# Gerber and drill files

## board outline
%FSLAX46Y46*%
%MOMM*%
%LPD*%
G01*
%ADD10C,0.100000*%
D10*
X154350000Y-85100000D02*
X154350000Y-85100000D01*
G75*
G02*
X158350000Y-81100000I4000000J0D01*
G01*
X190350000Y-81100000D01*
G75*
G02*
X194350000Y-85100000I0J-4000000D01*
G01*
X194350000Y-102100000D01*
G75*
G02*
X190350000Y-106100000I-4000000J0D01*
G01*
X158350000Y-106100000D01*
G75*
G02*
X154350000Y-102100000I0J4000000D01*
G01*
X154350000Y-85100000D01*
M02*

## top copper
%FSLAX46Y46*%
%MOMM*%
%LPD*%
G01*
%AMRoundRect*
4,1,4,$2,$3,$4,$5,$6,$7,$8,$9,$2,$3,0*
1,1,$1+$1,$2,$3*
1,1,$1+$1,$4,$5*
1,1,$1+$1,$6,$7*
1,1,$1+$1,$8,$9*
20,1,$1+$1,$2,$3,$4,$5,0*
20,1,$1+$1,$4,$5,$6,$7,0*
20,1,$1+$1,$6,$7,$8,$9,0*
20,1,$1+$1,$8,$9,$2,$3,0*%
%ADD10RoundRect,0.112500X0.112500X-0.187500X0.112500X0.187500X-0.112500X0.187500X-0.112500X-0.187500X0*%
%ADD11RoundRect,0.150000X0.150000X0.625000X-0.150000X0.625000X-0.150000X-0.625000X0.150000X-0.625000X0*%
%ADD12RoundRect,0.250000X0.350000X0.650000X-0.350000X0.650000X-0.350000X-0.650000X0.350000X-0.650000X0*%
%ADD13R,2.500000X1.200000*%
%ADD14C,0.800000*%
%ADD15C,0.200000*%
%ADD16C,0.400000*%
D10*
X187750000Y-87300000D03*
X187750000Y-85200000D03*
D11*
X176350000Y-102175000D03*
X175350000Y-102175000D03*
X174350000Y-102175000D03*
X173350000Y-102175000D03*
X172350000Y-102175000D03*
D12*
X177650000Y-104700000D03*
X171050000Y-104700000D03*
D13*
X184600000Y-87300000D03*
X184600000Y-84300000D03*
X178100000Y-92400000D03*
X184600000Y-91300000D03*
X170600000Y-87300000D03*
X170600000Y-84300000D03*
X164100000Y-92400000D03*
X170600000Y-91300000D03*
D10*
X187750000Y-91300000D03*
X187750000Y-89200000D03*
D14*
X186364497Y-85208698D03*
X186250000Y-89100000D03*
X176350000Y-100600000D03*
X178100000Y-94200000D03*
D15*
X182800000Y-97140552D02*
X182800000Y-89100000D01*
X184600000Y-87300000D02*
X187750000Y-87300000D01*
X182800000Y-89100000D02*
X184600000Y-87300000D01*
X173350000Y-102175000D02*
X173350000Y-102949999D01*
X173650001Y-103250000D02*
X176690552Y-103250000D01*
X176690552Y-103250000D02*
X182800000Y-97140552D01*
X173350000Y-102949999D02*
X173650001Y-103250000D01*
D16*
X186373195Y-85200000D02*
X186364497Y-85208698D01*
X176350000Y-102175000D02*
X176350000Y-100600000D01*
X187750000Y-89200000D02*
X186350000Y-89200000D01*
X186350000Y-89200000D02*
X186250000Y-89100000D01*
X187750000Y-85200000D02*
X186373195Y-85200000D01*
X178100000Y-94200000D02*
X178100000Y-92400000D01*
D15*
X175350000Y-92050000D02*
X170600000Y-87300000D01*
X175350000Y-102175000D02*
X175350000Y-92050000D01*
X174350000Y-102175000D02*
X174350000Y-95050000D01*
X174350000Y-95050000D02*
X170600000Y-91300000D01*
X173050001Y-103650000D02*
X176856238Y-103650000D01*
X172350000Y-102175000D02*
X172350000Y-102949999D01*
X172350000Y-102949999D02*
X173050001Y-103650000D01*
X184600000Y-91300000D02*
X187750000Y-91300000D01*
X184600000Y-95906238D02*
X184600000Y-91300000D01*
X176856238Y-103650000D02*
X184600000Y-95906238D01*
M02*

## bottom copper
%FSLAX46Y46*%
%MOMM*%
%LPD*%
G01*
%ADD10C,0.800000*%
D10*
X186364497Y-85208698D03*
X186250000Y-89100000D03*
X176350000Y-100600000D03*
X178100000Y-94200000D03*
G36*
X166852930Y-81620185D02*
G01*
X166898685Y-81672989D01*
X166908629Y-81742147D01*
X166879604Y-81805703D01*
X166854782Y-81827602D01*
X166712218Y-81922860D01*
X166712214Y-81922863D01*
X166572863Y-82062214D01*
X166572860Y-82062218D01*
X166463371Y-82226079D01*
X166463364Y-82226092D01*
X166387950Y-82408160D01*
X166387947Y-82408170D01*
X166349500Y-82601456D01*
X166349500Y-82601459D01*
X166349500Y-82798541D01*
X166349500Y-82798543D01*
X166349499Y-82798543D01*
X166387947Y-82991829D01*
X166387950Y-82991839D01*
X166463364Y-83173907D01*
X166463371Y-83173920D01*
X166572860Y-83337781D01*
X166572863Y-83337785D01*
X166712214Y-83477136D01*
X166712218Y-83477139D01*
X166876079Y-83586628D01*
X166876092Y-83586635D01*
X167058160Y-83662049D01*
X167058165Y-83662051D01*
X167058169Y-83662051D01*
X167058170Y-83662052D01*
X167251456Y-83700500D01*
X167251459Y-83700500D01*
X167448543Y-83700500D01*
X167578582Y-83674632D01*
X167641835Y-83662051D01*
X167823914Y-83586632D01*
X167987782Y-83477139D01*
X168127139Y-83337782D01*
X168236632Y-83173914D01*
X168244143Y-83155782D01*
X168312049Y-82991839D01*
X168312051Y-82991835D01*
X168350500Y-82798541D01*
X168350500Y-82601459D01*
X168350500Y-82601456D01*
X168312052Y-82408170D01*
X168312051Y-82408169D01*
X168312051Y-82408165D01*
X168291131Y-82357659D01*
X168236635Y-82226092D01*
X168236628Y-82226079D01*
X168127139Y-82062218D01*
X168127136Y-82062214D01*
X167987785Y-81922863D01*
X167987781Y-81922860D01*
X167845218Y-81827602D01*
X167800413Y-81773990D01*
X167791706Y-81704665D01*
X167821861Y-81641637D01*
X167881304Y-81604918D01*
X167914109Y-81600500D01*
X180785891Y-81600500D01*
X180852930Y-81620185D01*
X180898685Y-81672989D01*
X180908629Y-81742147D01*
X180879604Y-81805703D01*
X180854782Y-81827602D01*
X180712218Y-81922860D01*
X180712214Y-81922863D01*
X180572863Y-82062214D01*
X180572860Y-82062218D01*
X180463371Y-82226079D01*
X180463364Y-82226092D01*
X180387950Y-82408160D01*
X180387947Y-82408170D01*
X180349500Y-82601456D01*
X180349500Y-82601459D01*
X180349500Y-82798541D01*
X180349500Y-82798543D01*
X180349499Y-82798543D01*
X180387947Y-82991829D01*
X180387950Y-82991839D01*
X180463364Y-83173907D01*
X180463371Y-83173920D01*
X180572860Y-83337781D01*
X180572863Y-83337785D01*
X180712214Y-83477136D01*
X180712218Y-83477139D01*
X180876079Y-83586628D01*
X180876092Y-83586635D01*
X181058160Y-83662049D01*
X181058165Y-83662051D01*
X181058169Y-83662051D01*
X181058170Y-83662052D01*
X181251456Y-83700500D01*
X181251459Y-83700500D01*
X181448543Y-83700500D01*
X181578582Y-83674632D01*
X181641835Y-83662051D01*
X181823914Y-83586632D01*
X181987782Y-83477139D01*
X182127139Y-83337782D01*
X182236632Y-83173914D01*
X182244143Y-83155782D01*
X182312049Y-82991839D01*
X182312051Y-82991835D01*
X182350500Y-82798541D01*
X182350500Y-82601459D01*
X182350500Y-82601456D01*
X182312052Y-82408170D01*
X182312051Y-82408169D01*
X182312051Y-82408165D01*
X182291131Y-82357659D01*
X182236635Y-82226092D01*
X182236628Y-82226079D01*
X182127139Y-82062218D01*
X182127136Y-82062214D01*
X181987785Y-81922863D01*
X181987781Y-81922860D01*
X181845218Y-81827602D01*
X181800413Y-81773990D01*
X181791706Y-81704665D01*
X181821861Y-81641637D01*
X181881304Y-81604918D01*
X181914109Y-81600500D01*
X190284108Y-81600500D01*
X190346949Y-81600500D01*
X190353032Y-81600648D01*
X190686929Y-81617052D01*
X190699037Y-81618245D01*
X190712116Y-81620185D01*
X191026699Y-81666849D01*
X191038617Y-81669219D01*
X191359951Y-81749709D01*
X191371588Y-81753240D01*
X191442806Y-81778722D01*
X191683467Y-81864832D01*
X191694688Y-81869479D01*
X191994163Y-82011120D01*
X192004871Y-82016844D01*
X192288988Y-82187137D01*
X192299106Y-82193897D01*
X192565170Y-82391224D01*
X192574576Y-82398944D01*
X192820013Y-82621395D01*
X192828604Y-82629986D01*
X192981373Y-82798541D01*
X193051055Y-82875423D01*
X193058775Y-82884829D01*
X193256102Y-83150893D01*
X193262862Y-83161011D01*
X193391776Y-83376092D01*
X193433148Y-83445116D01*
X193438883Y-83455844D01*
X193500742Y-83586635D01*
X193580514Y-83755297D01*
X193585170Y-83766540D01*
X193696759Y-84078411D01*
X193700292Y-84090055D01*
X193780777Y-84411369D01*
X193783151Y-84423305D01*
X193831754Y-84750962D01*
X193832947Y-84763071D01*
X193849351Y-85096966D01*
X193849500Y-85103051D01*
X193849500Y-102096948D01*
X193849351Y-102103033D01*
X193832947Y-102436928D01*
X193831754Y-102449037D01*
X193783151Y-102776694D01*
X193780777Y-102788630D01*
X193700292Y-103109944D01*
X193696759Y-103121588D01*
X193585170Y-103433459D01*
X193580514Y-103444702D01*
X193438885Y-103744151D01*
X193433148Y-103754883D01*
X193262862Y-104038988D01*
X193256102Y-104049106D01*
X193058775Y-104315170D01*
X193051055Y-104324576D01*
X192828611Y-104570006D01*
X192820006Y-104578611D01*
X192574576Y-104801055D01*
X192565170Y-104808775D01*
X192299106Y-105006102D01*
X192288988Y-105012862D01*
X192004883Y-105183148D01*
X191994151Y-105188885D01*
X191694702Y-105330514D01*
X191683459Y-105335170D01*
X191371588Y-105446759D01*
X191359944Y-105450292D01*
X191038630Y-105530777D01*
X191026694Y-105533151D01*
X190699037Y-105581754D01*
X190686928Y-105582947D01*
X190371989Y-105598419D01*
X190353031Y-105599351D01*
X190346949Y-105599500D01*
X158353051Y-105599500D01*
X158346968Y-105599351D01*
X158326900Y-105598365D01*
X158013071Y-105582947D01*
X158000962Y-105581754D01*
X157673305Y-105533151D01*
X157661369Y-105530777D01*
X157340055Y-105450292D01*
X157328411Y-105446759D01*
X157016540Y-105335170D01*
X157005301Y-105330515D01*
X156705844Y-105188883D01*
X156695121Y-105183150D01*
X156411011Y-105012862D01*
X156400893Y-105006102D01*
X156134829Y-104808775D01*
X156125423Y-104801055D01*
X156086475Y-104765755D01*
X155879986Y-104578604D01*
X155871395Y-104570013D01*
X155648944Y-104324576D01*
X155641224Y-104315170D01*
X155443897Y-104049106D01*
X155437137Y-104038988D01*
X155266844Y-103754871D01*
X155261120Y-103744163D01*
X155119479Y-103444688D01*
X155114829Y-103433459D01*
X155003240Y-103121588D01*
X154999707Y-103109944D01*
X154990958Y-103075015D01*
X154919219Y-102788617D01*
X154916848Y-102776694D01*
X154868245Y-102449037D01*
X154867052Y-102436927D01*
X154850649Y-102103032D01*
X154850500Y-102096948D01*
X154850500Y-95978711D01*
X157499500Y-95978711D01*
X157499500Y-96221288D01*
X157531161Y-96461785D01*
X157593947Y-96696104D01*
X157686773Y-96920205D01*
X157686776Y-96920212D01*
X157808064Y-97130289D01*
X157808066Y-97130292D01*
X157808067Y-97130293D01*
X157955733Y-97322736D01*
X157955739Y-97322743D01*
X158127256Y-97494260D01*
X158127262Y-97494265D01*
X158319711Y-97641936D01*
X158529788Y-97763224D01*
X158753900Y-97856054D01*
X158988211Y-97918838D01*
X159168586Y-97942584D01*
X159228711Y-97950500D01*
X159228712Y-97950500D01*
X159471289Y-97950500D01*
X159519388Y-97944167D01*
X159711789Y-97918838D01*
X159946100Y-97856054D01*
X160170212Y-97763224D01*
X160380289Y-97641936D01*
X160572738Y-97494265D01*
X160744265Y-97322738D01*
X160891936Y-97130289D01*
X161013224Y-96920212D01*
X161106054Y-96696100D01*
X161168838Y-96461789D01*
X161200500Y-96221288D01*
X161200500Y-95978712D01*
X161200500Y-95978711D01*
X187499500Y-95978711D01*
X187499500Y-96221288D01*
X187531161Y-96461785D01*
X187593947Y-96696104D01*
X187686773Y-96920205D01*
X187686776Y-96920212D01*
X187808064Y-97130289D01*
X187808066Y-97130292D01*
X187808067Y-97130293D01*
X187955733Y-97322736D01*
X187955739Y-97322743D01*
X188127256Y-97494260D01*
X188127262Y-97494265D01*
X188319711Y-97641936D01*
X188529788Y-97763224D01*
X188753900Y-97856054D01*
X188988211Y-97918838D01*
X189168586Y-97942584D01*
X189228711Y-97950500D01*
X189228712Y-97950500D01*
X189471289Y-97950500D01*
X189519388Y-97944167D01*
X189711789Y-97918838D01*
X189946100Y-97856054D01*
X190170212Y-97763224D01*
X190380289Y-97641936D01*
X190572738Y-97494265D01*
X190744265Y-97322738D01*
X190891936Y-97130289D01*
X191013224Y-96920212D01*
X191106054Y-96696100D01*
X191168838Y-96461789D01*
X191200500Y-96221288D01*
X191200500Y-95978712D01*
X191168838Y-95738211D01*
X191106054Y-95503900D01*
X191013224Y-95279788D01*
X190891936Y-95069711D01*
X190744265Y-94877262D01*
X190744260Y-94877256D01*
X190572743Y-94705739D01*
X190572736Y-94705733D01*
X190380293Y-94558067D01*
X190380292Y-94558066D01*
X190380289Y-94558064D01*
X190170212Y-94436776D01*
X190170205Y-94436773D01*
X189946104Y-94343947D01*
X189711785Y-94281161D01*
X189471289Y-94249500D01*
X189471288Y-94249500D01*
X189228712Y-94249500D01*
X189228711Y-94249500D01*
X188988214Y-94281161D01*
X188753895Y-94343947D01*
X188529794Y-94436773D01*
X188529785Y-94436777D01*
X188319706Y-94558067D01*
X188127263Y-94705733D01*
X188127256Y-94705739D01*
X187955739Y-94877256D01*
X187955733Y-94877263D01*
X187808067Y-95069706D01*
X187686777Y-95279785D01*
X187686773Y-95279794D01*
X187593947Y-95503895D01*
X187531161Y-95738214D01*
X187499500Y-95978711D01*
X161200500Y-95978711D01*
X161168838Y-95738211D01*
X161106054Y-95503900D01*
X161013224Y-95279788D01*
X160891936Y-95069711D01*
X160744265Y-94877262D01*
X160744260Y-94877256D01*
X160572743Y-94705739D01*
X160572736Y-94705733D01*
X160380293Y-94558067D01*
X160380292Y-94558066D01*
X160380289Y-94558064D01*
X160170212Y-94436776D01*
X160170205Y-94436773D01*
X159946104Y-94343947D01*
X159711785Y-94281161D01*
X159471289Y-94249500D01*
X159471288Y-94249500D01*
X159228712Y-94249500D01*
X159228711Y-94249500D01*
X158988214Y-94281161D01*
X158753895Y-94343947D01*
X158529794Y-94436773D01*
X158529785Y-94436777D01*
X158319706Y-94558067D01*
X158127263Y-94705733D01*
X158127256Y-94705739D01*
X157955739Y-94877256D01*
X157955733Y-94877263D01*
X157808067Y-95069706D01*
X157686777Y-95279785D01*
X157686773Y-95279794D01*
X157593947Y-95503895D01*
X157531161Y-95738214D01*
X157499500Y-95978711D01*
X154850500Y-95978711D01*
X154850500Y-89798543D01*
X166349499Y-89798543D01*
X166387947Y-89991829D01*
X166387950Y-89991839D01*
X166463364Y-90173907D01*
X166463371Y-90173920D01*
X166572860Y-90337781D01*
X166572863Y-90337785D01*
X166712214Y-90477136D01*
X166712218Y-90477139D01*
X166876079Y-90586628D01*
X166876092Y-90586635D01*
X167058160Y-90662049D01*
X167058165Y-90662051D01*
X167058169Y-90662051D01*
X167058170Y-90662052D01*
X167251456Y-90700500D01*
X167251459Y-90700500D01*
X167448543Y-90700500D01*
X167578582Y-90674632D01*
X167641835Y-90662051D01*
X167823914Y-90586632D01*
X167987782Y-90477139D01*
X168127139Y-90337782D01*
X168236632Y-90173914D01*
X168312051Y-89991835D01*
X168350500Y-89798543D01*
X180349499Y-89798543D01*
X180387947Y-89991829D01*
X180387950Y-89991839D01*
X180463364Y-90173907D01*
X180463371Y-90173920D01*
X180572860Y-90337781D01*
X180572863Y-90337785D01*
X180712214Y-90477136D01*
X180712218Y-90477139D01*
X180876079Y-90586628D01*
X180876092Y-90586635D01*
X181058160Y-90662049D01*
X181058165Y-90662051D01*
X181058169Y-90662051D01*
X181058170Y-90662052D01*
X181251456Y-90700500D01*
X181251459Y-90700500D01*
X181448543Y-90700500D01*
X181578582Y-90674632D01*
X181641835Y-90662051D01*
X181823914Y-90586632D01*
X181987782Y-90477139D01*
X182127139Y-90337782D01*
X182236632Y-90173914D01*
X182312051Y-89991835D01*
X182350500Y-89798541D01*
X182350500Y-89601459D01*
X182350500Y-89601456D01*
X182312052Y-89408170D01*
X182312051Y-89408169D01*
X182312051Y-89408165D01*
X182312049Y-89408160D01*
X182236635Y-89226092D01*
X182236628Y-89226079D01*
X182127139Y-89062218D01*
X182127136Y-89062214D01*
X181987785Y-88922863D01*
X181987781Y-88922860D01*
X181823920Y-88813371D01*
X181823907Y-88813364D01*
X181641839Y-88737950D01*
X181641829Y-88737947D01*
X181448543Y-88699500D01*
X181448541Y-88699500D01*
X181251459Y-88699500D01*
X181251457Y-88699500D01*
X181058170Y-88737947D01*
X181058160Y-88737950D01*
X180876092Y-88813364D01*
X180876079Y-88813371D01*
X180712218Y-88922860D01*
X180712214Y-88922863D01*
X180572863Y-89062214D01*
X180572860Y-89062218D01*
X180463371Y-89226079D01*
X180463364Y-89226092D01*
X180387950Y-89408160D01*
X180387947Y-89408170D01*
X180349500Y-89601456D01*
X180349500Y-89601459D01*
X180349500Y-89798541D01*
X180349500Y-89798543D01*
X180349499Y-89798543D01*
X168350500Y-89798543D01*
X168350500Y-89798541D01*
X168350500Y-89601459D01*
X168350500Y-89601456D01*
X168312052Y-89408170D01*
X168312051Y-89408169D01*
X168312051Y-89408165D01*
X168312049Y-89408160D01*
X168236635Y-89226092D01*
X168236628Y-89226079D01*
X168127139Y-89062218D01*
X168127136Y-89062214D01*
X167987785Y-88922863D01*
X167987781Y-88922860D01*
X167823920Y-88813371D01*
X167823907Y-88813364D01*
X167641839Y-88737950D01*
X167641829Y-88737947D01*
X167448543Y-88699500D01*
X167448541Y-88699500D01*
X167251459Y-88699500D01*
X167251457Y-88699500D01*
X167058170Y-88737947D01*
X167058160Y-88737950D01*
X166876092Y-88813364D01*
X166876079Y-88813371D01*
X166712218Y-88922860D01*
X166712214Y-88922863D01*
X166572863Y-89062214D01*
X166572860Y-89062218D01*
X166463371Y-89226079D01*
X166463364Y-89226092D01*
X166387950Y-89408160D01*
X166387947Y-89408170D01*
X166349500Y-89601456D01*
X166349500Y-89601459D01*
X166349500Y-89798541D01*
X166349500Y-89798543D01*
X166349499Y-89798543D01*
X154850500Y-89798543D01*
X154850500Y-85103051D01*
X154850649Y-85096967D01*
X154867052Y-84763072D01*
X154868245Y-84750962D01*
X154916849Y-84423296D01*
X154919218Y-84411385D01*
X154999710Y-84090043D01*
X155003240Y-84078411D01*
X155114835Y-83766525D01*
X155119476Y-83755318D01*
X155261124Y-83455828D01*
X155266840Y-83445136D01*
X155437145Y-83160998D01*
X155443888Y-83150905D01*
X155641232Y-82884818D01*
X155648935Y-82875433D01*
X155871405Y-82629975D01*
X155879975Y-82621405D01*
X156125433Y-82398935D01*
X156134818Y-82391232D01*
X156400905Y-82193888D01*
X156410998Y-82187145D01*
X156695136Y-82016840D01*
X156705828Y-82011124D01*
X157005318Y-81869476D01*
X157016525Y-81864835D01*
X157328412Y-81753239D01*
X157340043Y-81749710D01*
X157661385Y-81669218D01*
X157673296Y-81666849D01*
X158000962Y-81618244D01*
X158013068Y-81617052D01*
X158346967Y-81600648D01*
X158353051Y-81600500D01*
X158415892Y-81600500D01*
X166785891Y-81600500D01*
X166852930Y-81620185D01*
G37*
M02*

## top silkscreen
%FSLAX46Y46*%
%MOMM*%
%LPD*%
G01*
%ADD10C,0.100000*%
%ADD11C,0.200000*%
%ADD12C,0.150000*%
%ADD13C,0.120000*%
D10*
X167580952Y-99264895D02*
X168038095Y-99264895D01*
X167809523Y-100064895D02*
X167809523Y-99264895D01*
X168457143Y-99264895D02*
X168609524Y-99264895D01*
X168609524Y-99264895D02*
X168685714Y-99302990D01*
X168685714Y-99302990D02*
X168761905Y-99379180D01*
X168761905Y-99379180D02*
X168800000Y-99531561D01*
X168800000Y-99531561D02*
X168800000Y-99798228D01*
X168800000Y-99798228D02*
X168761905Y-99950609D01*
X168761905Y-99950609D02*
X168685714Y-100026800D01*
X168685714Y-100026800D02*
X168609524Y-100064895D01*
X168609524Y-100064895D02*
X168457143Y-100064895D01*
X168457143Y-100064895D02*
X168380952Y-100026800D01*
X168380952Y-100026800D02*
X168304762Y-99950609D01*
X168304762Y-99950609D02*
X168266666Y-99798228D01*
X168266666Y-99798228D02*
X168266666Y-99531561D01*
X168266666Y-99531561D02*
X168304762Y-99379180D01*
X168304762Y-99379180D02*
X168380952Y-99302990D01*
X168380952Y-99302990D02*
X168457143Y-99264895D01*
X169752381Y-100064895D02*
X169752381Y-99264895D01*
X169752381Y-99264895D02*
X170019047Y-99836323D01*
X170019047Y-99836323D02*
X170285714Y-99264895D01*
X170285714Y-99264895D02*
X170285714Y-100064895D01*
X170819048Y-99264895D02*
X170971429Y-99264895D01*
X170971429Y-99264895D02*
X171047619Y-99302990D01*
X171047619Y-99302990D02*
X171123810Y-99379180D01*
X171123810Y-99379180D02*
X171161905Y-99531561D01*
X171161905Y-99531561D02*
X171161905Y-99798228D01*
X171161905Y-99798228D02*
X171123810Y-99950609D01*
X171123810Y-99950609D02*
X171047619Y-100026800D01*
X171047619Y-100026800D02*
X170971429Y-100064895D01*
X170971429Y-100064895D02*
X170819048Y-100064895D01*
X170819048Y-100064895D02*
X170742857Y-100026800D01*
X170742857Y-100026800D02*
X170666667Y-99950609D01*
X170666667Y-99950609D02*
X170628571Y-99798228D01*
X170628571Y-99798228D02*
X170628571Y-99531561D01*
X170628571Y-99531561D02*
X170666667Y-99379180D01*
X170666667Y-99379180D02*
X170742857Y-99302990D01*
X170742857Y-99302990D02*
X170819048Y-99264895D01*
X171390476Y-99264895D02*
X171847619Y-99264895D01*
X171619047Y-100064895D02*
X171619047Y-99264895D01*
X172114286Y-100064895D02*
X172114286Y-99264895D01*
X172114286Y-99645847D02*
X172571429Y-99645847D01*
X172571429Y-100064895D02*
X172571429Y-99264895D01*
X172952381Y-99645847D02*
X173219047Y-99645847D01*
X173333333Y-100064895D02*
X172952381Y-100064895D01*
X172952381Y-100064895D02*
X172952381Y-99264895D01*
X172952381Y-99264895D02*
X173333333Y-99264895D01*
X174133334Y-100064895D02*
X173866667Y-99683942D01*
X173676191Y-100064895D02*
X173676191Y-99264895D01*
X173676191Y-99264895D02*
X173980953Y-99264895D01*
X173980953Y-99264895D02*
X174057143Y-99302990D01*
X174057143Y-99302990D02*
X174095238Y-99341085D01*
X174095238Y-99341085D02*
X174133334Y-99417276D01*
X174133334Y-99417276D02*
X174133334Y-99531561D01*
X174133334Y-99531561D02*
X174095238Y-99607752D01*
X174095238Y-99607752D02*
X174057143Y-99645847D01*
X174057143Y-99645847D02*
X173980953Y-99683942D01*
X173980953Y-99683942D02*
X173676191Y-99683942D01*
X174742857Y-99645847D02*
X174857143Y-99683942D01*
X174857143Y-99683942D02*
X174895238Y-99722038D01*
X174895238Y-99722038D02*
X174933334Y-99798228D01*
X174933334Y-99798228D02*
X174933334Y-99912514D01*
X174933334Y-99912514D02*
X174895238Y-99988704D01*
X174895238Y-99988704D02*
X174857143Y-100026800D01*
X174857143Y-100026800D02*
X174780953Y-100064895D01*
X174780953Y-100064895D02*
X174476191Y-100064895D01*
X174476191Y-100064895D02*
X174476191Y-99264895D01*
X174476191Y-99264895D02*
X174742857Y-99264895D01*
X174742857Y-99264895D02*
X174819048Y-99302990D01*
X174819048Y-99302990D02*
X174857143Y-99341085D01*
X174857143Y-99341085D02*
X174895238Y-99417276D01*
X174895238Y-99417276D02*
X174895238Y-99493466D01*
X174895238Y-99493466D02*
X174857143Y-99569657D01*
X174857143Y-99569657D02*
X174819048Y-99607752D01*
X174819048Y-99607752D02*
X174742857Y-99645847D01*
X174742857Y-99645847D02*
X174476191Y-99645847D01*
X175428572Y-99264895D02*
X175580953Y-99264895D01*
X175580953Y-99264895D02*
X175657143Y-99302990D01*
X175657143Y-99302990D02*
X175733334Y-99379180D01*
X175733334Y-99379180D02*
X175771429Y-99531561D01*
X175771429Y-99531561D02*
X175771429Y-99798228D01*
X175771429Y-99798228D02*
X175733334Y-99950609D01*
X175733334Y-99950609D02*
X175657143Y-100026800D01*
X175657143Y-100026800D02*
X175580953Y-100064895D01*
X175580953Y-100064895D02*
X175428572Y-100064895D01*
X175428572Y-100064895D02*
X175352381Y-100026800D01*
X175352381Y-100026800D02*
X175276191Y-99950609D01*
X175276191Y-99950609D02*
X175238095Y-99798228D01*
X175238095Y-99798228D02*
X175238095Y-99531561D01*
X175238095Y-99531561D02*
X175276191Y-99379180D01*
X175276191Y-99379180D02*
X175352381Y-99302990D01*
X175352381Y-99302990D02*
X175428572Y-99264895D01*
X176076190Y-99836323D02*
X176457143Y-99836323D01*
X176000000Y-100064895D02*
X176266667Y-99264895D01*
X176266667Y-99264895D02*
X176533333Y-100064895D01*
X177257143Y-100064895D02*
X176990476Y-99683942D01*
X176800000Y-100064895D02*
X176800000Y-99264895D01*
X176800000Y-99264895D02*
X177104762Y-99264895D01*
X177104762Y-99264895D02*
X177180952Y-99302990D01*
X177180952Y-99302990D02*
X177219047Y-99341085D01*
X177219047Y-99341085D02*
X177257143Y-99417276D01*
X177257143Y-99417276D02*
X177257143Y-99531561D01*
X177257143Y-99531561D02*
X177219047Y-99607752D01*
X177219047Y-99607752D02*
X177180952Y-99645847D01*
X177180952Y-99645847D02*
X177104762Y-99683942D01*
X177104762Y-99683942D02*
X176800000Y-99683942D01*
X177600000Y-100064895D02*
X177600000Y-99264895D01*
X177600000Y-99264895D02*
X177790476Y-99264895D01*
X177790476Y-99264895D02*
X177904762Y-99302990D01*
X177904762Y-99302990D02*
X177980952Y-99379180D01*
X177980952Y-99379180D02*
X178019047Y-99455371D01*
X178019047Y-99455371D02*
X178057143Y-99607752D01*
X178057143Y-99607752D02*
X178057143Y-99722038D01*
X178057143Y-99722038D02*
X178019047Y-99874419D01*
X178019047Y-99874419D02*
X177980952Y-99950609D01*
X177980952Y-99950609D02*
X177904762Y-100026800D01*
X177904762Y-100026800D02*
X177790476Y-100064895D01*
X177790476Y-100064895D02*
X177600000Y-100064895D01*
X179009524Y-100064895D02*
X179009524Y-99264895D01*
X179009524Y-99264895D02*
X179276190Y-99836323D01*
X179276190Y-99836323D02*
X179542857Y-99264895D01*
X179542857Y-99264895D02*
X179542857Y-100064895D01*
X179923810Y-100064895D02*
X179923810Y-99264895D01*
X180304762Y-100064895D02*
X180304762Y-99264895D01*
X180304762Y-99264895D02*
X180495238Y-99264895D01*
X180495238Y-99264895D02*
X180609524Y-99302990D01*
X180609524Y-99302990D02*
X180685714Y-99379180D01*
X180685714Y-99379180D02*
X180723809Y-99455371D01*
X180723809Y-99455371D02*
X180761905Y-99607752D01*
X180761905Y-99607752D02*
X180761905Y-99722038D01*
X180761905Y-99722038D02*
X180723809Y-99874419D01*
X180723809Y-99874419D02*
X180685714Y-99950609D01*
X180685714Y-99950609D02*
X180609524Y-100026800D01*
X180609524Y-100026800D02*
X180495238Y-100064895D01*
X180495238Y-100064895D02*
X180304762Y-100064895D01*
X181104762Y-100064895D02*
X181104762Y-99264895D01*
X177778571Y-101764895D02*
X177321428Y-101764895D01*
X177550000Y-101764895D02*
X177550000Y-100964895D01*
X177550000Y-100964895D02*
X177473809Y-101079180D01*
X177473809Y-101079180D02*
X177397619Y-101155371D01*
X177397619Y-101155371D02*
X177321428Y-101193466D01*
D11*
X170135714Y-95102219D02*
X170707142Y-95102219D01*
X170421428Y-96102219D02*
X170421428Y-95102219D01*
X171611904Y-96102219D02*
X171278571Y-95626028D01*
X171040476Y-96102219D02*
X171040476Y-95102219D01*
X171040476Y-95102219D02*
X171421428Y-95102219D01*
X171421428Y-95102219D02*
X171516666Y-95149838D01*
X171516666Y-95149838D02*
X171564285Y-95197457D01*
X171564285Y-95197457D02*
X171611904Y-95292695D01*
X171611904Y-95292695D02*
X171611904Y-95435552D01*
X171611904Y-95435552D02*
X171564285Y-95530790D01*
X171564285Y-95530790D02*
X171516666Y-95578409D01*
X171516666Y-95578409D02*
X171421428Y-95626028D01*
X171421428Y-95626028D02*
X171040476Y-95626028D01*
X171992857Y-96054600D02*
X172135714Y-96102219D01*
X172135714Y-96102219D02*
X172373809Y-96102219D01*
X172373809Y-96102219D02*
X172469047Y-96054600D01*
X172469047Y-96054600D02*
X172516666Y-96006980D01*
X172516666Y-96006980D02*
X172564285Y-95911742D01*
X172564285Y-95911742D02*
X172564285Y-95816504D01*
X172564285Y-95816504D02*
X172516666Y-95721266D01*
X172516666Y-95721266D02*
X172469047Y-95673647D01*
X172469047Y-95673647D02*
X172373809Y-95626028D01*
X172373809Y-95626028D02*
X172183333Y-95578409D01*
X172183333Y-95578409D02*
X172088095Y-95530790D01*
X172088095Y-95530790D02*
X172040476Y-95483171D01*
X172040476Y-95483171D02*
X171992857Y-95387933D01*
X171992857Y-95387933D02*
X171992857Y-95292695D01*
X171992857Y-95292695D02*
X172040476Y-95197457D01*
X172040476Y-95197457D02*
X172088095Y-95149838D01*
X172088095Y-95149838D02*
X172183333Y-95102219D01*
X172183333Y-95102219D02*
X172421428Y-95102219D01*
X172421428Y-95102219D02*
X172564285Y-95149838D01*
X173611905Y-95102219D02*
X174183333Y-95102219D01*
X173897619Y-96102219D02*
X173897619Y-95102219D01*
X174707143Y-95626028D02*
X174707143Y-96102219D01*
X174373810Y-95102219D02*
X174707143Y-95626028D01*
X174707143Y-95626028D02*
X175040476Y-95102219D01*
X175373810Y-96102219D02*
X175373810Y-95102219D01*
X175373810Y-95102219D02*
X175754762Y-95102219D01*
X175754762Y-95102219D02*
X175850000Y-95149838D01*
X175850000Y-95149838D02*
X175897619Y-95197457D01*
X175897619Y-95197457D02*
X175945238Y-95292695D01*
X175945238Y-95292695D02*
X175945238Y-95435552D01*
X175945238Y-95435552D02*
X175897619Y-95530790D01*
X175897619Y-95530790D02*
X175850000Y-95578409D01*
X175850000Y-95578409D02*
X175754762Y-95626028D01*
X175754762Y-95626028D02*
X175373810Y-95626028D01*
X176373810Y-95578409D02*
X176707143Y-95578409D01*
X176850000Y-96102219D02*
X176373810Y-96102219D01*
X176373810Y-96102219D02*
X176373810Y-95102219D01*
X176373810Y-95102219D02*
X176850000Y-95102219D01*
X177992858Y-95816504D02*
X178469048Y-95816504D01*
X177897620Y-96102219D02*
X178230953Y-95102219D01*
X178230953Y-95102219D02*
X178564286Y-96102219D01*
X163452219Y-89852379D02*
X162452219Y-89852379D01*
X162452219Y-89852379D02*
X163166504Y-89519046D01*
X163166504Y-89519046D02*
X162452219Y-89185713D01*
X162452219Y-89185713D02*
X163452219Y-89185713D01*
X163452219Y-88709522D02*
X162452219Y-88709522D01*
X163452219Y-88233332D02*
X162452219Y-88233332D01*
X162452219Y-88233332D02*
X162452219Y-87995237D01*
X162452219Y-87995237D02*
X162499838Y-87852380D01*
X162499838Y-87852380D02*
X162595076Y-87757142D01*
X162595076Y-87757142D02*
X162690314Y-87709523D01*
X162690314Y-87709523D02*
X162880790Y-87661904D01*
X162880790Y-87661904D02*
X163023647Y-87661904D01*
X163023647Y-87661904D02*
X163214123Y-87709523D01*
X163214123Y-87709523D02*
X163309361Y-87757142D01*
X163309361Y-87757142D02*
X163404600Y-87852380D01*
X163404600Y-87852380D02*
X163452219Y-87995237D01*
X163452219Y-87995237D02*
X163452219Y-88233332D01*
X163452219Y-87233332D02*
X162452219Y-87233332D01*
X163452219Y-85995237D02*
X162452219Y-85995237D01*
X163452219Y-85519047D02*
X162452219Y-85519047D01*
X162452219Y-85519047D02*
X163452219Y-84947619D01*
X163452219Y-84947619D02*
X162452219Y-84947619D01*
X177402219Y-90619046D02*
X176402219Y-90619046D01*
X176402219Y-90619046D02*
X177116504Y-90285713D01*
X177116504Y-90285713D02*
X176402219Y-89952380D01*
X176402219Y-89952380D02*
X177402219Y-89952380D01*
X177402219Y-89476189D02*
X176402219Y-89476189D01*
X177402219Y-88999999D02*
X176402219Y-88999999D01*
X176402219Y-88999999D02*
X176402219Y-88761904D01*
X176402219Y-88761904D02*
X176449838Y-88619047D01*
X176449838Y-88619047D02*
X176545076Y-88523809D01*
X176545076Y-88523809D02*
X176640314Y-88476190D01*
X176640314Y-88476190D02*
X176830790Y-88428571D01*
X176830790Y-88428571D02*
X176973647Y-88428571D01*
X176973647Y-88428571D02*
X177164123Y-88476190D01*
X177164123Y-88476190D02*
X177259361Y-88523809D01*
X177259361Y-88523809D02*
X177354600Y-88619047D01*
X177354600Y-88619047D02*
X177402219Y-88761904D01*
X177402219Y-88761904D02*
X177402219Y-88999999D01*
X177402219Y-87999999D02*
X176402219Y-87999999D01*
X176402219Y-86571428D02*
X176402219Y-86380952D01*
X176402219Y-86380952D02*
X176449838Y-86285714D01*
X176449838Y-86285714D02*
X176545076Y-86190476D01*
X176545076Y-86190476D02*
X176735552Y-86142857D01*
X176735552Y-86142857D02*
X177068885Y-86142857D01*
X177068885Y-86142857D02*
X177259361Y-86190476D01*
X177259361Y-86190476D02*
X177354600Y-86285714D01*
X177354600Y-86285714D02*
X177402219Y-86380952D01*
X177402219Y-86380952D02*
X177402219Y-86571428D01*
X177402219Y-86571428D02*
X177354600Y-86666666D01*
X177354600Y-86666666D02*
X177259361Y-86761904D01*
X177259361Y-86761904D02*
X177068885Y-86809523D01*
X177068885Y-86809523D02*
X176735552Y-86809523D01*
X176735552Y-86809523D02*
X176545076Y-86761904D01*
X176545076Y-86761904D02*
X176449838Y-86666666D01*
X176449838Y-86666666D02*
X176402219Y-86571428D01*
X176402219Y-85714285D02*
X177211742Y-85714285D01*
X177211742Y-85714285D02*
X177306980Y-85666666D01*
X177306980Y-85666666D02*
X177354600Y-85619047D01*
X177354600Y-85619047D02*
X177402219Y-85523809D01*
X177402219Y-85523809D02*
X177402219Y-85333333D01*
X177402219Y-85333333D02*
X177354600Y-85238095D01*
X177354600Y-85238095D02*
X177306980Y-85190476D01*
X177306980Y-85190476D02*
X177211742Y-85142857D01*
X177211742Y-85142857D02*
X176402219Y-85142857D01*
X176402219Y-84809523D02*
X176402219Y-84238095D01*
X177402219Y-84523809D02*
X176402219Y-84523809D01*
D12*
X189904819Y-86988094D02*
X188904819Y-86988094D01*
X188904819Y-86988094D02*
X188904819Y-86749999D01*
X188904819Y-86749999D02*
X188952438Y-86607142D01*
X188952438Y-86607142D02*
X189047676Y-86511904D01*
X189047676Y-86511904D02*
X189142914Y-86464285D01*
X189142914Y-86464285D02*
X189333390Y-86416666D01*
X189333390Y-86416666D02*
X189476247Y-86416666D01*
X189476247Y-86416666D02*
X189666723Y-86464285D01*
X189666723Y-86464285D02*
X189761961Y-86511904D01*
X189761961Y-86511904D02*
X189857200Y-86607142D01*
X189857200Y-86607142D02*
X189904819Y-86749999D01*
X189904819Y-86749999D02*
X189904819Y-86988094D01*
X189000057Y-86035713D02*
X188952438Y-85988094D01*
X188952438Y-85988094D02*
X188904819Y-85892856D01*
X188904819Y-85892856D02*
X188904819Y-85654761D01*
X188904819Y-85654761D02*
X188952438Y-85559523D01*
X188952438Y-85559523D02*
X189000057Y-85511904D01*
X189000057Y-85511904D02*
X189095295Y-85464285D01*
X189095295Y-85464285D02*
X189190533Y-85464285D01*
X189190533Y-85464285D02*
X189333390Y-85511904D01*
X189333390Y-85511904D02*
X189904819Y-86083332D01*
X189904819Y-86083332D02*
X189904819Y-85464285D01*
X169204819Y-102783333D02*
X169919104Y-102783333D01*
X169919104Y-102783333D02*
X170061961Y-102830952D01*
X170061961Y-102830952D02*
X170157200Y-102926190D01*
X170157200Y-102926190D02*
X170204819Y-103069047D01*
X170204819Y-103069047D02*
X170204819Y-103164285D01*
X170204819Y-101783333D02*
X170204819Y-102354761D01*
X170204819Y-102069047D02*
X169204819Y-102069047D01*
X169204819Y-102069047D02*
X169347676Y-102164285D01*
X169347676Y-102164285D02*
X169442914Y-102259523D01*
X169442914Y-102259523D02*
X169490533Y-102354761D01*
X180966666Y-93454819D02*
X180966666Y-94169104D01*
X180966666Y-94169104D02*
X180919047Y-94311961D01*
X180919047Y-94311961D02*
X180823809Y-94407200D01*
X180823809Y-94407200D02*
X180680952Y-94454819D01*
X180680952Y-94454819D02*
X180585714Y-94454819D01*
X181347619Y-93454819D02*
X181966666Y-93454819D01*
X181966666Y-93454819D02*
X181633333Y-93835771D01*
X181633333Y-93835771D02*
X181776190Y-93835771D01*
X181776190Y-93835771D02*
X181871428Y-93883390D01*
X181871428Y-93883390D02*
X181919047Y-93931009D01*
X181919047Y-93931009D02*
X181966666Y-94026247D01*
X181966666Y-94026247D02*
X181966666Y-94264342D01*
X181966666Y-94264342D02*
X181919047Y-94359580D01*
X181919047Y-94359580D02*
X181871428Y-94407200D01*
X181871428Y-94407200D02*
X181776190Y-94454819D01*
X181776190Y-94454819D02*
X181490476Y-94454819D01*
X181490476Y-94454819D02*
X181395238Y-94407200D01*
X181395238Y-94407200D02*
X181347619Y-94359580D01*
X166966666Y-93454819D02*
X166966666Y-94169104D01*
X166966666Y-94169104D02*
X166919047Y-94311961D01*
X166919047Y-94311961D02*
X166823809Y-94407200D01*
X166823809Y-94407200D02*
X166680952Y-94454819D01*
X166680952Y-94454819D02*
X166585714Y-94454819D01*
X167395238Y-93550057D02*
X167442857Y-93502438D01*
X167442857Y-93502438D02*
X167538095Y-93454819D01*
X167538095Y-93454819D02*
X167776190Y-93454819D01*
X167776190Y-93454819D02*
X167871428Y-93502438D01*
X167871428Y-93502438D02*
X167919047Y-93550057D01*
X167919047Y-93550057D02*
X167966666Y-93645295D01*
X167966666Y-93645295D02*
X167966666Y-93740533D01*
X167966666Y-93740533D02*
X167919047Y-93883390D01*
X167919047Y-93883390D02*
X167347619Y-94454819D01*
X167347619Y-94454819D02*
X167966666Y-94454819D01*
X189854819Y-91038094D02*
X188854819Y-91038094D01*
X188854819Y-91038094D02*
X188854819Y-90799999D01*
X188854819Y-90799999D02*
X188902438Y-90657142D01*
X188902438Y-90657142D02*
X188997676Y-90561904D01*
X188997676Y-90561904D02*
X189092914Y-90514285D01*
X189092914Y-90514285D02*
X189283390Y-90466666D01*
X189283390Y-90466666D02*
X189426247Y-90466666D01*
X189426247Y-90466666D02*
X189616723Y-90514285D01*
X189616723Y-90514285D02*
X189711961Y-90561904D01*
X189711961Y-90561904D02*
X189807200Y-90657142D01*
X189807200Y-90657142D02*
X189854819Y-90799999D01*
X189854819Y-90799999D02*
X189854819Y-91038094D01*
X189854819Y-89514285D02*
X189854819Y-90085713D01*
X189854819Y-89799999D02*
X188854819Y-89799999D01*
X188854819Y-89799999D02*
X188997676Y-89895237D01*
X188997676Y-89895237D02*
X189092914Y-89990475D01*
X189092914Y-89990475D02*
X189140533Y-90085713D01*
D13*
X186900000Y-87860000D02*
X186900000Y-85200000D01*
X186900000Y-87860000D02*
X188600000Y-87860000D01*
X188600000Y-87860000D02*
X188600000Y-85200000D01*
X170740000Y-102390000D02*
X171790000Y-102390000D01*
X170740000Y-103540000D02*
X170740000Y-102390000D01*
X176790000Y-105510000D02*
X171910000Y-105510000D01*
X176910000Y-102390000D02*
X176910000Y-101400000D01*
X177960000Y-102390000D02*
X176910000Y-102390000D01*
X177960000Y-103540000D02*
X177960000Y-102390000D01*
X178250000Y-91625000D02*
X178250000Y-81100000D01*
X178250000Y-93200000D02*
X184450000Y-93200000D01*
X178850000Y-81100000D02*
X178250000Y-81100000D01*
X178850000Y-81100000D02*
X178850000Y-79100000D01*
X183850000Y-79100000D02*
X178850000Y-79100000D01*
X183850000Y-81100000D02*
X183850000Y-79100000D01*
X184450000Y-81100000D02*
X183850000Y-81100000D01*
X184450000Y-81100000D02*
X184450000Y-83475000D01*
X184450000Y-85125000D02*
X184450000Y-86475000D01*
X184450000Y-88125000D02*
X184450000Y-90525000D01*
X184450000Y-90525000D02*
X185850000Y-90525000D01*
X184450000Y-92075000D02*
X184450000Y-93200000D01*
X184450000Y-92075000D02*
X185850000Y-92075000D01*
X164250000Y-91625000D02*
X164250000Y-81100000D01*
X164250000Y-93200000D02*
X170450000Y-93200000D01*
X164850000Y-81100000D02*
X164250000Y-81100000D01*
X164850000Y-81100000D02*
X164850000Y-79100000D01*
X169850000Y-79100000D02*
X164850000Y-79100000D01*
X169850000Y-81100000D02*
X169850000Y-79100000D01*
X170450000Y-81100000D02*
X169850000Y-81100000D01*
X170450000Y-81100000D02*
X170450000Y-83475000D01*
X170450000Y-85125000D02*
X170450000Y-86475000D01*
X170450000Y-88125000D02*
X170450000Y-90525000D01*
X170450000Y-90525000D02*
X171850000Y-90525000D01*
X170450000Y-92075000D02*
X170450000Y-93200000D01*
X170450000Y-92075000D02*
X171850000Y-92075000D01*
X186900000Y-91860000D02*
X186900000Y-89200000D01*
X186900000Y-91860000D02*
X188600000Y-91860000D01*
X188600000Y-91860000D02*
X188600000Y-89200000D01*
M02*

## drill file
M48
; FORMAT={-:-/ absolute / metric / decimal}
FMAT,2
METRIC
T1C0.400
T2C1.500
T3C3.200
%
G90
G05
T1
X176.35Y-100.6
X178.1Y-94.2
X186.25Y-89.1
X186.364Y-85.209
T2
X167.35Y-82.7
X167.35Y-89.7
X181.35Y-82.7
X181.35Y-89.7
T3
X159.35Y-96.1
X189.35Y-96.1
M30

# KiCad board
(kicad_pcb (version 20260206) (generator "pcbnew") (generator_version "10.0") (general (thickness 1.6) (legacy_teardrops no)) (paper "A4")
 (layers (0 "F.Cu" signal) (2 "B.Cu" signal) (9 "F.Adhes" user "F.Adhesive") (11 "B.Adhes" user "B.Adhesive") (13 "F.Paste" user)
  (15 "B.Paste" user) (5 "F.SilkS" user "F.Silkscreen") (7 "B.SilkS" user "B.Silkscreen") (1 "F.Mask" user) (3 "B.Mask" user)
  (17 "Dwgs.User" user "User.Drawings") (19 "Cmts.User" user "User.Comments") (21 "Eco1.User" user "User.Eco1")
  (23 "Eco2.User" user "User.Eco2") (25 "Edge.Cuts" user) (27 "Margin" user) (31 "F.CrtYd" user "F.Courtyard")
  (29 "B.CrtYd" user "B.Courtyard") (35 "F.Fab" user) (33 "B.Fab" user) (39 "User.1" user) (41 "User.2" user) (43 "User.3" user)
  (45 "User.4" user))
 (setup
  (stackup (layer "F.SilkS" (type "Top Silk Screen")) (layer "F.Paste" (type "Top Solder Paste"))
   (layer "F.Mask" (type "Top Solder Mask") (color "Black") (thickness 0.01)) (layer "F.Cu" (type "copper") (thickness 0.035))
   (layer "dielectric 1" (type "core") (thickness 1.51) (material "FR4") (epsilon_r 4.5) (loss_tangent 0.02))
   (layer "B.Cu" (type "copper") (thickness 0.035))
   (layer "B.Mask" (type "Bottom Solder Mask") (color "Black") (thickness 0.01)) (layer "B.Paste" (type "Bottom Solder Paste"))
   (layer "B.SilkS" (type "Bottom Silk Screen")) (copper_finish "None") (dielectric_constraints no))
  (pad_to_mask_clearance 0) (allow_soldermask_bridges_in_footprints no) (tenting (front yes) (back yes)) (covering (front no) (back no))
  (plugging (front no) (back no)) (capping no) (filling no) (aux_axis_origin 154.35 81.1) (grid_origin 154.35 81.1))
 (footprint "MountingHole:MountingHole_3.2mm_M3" (layer "F.Cu") (at 159.35 96.1)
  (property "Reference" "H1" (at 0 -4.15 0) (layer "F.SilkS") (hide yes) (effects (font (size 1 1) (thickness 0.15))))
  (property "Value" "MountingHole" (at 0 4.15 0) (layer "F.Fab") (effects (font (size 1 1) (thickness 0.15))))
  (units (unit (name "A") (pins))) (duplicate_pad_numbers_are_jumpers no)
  (pad "" np_thru_hole circle (at 0 0) (size 3.2 3.2) (drill 3.2) (layers "*.Cu" "*.Mask")))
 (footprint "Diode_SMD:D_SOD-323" (layer "F.Cu") (at 187.75 86.25 90)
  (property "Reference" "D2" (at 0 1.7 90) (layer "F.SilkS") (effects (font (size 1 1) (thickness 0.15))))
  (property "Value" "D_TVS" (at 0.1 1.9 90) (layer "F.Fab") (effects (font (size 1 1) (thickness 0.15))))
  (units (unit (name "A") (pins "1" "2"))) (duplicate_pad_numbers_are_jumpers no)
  (fp_line (start -1.61 -0.85) (end 1.05 -0.85) (stroke (width 0.12) (type solid)) (layer "F.SilkS"))
  (fp_line (start -1.61 -0.85) (end -1.61 0.85) (stroke (width 0.12) (type solid)) (layer "F.SilkS"))
  (fp_line (start -1.61 0.85) (end 1.05 0.85) (stroke (width 0.12) (type solid)) (layer "F.SilkS"))
  (pad "1" smd roundrect (at -1.05 0 90) (size 0.6 0.45) (layers "F.Cu" "F.Mask" "F.Paste") (roundrect_rratio 0.25) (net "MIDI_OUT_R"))
  (pad "2" smd roundrect (at 1.05 0 90) (size 0.6 0.45) (layers "F.Cu" "F.Mask" "F.Paste") (roundrect_rratio 0.25) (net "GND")))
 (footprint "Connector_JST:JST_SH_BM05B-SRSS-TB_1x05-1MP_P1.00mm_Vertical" (layer "F.Cu") (at 174.35 103.5 180)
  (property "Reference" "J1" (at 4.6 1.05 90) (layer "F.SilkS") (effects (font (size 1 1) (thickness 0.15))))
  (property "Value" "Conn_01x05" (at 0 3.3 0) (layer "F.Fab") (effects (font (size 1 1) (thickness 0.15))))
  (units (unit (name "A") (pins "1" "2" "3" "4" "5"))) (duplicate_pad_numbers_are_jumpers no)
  (fp_line (start 3.61 1.11) (end 2.56 1.11) (stroke (width 0.12) (type solid)) (layer "F.SilkS"))
  (fp_line (start 3.61 -0.04) (end 3.61 1.11) (stroke (width 0.12) (type solid)) (layer "F.SilkS"))
  (fp_line (start -2.44 -2.01) (end 2.44 -2.01) (stroke (width 0.12) (type solid)) (layer "F.SilkS"))
  (fp_line (start -2.56 1.11) (end -2.56 2.1) (stroke (width 0.12) (type solid)) (layer "F.SilkS"))
  (fp_line (start -3.61 1.11) (end -2.56 1.11) (stroke (width 0.12) (type solid)) (layer "F.SilkS"))
  (fp_line (start -3.61 -0.04) (end -3.61 1.11) (stroke (width 0.12) (type solid)) (layer "F.SilkS"))
  (pad "1" smd roundrect (at -2 1.325 180) (size 0.6 1.55) (layers "F.Cu" "F.Mask" "F.Paste") (roundrect_rratio 0.25) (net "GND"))
  (pad "2" smd roundrect (at -1 1.325 180) (size 0.6 1.55) (layers "F.Cu" "F.Mask" "F.Paste") (roundrect_rratio 0.25) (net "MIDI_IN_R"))
  (pad "3" smd roundrect (at 0 1.325 180) (size 0.6 1.55) (layers "F.Cu" "F.Mask" "F.Paste") (roundrect_rratio 0.25) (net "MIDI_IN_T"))
  (pad "4" smd roundrect (at 1 1.325 180) (size 0.6 1.55) (layers "F.Cu" "F.Mask" "F.Paste") (roundrect_rratio 0.25) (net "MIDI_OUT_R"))
  (pad "5" smd roundrect (at 2 1.325 180) (size 0.6 1.55) (layers "F.Cu" "F.Mask" "F.Paste") (roundrect_rratio 0.25) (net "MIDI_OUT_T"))
  (pad "MP" smd roundrect (at -3.3 -1.2 180) (size 1.2 1.8) (layers "F.Cu" "F.Mask" "F.Paste") (roundrect_rratio 0.208333))
  (pad "MP" smd roundrect (at 3.3 -1.2 180) (size 1.2 1.8) (layers "F.Cu" "F.Mask" "F.Paste") (roundrect_rratio 0.208333)))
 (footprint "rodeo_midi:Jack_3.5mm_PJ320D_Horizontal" (layer "F.Cu") (at 181.35 87.475 -90)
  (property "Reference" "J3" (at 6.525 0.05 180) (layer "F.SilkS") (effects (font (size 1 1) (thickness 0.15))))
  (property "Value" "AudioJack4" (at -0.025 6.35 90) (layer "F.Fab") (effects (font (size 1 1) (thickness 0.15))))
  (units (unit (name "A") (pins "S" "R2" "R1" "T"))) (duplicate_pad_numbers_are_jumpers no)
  (fp_line (start 4.15 3.1) (end -6.375 3.1) (stroke (width 0.12) (type solid)) (layer "F.SilkS"))
  (fp_line (start 5.725 3.1) (end 5.725 -3.1) (stroke (width 0.12) (type solid)) (layer "F.SilkS"))
  (fp_line (start -6.375 2.5) (end -6.375 3.1) (stroke (width 0.12) (type solid)) (layer "F.SilkS"))
  (fp_line (start -6.375 2.5) (end -8.375 2.5) (stroke (width 0.12) (type solid)) (layer "F.SilkS"))
  (fp_line (start -8.375 -2.5) (end -8.375 2.5) (stroke (width 0.12) (type solid)) (layer "F.SilkS"))
  (fp_line (start -6.375 -2.5) (end -8.375 -2.5) (stroke (width 0.12) (type solid)) (layer "F.SilkS"))
  (fp_line (start -6.375 -3.1) (end -6.375 -2.5) (stroke (width 0.12) (type solid)) (layer "F.SilkS"))
  (fp_line (start -6.375 -3.1) (end -4 -3.1) (stroke (width 0.12) (type solid)) (layer "F.SilkS"))
  (fp_line (start -2.35 -3.1) (end -1 -3.1) (stroke (width 0.12) (type solid)) (layer "F.SilkS"))
  (fp_line (start 0.65 -3.1) (end 3.05 -3.1) (stroke (width 0.12) (type solid)) (layer "F.SilkS"))
  (fp_line (start 3.05 -3.1) (end 3.05 -4.5) (stroke (width 0.12) (type solid)) (layer "F.SilkS"))
  (fp_line (start 4.6 -3.1) (end 5.725 -3.1) (stroke (width 0.12) (type solid)) (layer "F.SilkS"))
  (fp_line (start 4.6 -3.1) (end 4.6 -4.5) (stroke (width 0.12) (type solid)) (layer "F.SilkS"))
  (pad "" np_thru_hole circle (at -4.775 0 270) (size 1.5 1.5) (drill 1.5) (layers "*.Cu" "*.Mask"))
  (pad "" np_thru_hole circle (at 2.225 0 270) (size 1.5 1.5) (drill 1.5) (layers "*.Cu" "*.Mask"))
  (pad "R1" smd rect (at -0.175 -3.25 270) (size 1.2 2.5) (layers "F.Cu" "F.Mask" "F.Paste") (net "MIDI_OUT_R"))
  (pad "R2" smd rect (at -3.175 -3.25 270) (size 1.2 2.5) (layers "F.Cu" "F.Mask" "F.Paste") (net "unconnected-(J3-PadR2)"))
  (pad "S" smd rect (at 4.925 3.25 270) (size 1.2 2.5) (layers "F.Cu" "F.Mask" "F.Paste") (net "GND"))
  (pad "T" smd rect (at 3.825 -3.25 270) (size 1.2 2.5) (layers "F.Cu" "F.Mask" "F.Paste") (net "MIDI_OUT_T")))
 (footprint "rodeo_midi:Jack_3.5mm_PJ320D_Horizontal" (layer "F.Cu") (at 167.35 87.475 -90)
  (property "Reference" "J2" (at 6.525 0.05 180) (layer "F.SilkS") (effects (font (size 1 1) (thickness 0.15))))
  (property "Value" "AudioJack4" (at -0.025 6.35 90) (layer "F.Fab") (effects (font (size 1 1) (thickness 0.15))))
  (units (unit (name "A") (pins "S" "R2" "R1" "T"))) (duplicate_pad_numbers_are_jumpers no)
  (fp_line (start 4.15 3.1) (end -6.375 3.1) (stroke (width 0.12) (type solid)) (layer "F.SilkS"))
  (fp_line (start 5.725 3.1) (end 5.725 -3.1) (stroke (width 0.12) (type solid)) (layer "F.SilkS"))
  (fp_line (start -6.375 2.5) (end -6.375 3.1) (stroke (width 0.12) (type solid)) (layer "F.SilkS"))
  (fp_line (start -6.375 2.5) (end -8.375 2.5) (stroke (width 0.12) (type solid)) (layer "F.SilkS"))
  (fp_line (start -8.375 -2.5) (end -8.375 2.5) (stroke (width 0.12) (type solid)) (layer "F.SilkS"))
  (fp_line (start -6.375 -2.5) (end -8.375 -2.5) (stroke (width 0.12) (type solid)) (layer "F.SilkS"))
  (fp_line (start -6.375 -3.1) (end -6.375 -2.5) (stroke (width 0.12) (type solid)) (layer "F.SilkS"))
  (fp_line (start -6.375 -3.1) (end -4 -3.1) (stroke (width 0.12) (type solid)) (layer "F.SilkS"))
  (fp_line (start -2.35 -3.1) (end -1 -3.1) (stroke (width 0.12) (type solid)) (layer "F.SilkS"))
  (fp_line (start 0.65 -3.1) (end 3.05 -3.1) (stroke (width 0.12) (type solid)) (layer "F.SilkS"))
  (fp_line (start 3.05 -3.1) (end 3.05 -4.5) (stroke (width 0.12) (type solid)) (layer "F.SilkS"))
  (fp_line (start 4.6 -3.1) (end 5.725 -3.1) (stroke (width 0.12) (type solid)) (layer "F.SilkS"))
  (fp_line (start 4.6 -3.1) (end 4.6 -4.5) (stroke (width 0.12) (type solid)) (layer "F.SilkS"))
  (pad "" np_thru_hole circle (at -4.775 0 270) (size 1.5 1.5) (drill 1.5) (layers "*.Cu" "*.Mask"))
  (pad "" np_thru_hole circle (at 2.225 0 270) (size 1.5 1.5) (drill 1.5) (layers "*.Cu" "*.Mask"))
  (pad "R1" smd rect (at -0.175 -3.25 270) (size 1.2 2.5) (layers "F.Cu" "F.Mask" "F.Paste") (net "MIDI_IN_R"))
  (pad "R2" smd rect (at -3.175 -3.25 270) (size 1.2 2.5) (layers "F.Cu" "F.Mask" "F.Paste") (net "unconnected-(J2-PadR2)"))
  (pad "S" smd rect (at 4.925 3.25 270) (size 1.2 2.5) (layers "F.Cu" "F.Mask" "F.Paste") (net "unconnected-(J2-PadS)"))
  (pad "T" smd rect (at 3.825 -3.25 270) (size 1.2 2.5) (layers "F.Cu" "F.Mask" "F.Paste") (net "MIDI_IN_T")))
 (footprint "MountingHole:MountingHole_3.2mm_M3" (layer "F.Cu") (at 189.35 96.1)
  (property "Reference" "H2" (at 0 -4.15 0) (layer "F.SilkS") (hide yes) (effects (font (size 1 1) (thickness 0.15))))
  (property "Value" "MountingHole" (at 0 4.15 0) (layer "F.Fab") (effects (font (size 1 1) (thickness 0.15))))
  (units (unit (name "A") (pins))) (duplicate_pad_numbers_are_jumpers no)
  (pad "" np_thru_hole circle (at 0 0) (size 3.2 3.2) (drill 3.2) (layers "*.Cu" "*.Mask")))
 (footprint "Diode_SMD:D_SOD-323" (layer "F.Cu") (at 187.75 90.25 90)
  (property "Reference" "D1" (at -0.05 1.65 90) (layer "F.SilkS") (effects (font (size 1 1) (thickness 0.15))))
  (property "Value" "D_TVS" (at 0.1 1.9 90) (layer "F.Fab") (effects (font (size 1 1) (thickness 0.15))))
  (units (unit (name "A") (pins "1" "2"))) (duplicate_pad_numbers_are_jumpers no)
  (fp_line (start -1.61 -0.85) (end 1.05 -0.85) (stroke (width 0.12) (type solid)) (layer "F.SilkS"))
  (fp_line (start -1.61 -0.85) (end -1.61 0.85) (stroke (width 0.12) (type solid)) (layer "F.SilkS"))
  (fp_line (start -1.61 0.85) (end 1.05 0.85) (stroke (width 0.12) (type solid)) (layer "F.SilkS"))
  (pad "1" smd roundrect (at -1.05 0 90) (size 0.6 0.45) (layers "F.Cu" "F.Mask" "F.Paste") (roundrect_rratio 0.25) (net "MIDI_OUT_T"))
  (pad "2" smd roundrect (at 1.05 0 90) (size 0.6 0.45) (layers "F.Cu" "F.Mask" "F.Paste") (roundrect_rratio 0.25) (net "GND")))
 (gr_rect (start 154.35 81.1) (end 194.35 106.1) (radius 4) (stroke (width 0.1) (type solid)) (fill no) (layer "Edge.Cuts"))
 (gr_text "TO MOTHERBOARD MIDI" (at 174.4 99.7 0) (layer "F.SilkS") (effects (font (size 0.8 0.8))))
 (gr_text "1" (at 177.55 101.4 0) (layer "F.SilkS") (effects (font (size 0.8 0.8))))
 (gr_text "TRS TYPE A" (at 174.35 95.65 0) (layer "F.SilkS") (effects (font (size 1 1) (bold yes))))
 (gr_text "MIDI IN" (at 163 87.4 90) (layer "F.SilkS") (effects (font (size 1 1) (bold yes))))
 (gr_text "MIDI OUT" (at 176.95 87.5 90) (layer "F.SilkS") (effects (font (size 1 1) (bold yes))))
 (segment (start 182.8 97.140552) (end 182.8 89.1) (width 0.2) (layer "F.Cu") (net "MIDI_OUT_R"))
 (segment (start 184.6 87.3) (end 187.75 87.3) (width 0.2) (layer "F.Cu") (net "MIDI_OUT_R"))
 (segment (start 182.8 89.1) (end 184.6 87.3) (width 0.2) (layer "F.Cu") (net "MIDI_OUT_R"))
 (segment (start 173.35 102.175) (end 173.35 102.949999) (width 0.2) (layer "F.Cu") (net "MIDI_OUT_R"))
 (segment (start 173.650001 103.25) (end 176.690552 103.25) (width 0.2) (layer "F.Cu") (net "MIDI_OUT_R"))
 (segment (start 176.690552 103.25) (end 182.8 97.140552) (width 0.2) (layer "F.Cu") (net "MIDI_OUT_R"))
 (segment (start 173.35 102.949999) (end 173.650001 103.25) (width 0.2) (layer "F.Cu") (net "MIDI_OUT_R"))
 (segment (start 186.373195 85.2) (end 186.364497 85.208698) (width 0.4) (layer "F.Cu") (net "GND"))
 (segment (start 176.35 102.175) (end 176.35 100.6) (width 0.4) (layer "F.Cu") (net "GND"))
 (segment (start 187.75 89.2) (end 186.35 89.2) (width 0.4) (layer "F.Cu") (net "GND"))
 (segment (start 186.35 89.2) (end 186.25 89.1) (width 0.4) (layer "F.Cu") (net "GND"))
 (segment (start 187.75 85.2) (end 186.373195 85.2) (width 0.4) (layer "F.Cu") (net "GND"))
 (segment (start 178.1 94.2) (end 178.1 92.4) (width 0.4) (layer "F.Cu") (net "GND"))
 (via (at 186.364497 85.208698) (size 0.8) (drill 0.4) (layers "F.Cu" "B.Cu") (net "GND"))
 (via (at 186.25 89.1) (size 0.8) (drill 0.4) (layers "F.Cu" "B.Cu") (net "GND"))
 (via (at 176.35 100.6) (size 0.8) (drill 0.4) (layers "F.Cu" "B.Cu") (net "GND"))
 (via (at 178.1 94.2) (size 0.8) (drill 0.4) (layers "F.Cu" "B.Cu") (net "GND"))
 (segment (start 175.35 92.05) (end 170.6 87.3) (width 0.2) (layer "F.Cu") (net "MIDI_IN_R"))
 (segment (start 175.35 102.175) (end 175.35 92.05) (width 0.2) (layer "F.Cu") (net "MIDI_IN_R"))
 (segment (start 174.35 102.175) (end 174.35 95.05) (width 0.2) (layer "F.Cu") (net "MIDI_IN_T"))
 (segment (start 174.35 95.05) (end 170.6 91.3) (width 0.2) (layer "F.Cu") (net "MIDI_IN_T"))
 (segment (start 173.050001 103.65) (end 176.856238 103.65) (width 0.2) (layer "F.Cu") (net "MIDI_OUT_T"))
 (segment (start 172.35 102.175) (end 172.35 102.949999) (width 0.2) (layer "F.Cu") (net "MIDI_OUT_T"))
 (segment (start 172.35 102.949999) (end 173.050001 103.65) (width 0.2) (layer "F.Cu") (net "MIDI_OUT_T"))
 (segment (start 184.6 91.3) (end 187.75 91.3) (width 0.2) (layer "F.Cu") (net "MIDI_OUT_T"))
 (segment (start 184.6 95.906238) (end 184.6 91.3) (width 0.2) (layer "F.Cu") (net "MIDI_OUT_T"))
 (segment (start 176.856238 103.65) (end 184.6 95.906238) (width 0.2) (layer "F.Cu") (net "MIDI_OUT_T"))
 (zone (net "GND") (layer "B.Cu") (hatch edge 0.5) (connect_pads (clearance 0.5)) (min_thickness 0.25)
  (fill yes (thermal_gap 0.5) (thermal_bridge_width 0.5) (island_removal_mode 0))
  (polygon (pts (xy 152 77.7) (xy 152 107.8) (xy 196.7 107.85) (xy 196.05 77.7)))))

